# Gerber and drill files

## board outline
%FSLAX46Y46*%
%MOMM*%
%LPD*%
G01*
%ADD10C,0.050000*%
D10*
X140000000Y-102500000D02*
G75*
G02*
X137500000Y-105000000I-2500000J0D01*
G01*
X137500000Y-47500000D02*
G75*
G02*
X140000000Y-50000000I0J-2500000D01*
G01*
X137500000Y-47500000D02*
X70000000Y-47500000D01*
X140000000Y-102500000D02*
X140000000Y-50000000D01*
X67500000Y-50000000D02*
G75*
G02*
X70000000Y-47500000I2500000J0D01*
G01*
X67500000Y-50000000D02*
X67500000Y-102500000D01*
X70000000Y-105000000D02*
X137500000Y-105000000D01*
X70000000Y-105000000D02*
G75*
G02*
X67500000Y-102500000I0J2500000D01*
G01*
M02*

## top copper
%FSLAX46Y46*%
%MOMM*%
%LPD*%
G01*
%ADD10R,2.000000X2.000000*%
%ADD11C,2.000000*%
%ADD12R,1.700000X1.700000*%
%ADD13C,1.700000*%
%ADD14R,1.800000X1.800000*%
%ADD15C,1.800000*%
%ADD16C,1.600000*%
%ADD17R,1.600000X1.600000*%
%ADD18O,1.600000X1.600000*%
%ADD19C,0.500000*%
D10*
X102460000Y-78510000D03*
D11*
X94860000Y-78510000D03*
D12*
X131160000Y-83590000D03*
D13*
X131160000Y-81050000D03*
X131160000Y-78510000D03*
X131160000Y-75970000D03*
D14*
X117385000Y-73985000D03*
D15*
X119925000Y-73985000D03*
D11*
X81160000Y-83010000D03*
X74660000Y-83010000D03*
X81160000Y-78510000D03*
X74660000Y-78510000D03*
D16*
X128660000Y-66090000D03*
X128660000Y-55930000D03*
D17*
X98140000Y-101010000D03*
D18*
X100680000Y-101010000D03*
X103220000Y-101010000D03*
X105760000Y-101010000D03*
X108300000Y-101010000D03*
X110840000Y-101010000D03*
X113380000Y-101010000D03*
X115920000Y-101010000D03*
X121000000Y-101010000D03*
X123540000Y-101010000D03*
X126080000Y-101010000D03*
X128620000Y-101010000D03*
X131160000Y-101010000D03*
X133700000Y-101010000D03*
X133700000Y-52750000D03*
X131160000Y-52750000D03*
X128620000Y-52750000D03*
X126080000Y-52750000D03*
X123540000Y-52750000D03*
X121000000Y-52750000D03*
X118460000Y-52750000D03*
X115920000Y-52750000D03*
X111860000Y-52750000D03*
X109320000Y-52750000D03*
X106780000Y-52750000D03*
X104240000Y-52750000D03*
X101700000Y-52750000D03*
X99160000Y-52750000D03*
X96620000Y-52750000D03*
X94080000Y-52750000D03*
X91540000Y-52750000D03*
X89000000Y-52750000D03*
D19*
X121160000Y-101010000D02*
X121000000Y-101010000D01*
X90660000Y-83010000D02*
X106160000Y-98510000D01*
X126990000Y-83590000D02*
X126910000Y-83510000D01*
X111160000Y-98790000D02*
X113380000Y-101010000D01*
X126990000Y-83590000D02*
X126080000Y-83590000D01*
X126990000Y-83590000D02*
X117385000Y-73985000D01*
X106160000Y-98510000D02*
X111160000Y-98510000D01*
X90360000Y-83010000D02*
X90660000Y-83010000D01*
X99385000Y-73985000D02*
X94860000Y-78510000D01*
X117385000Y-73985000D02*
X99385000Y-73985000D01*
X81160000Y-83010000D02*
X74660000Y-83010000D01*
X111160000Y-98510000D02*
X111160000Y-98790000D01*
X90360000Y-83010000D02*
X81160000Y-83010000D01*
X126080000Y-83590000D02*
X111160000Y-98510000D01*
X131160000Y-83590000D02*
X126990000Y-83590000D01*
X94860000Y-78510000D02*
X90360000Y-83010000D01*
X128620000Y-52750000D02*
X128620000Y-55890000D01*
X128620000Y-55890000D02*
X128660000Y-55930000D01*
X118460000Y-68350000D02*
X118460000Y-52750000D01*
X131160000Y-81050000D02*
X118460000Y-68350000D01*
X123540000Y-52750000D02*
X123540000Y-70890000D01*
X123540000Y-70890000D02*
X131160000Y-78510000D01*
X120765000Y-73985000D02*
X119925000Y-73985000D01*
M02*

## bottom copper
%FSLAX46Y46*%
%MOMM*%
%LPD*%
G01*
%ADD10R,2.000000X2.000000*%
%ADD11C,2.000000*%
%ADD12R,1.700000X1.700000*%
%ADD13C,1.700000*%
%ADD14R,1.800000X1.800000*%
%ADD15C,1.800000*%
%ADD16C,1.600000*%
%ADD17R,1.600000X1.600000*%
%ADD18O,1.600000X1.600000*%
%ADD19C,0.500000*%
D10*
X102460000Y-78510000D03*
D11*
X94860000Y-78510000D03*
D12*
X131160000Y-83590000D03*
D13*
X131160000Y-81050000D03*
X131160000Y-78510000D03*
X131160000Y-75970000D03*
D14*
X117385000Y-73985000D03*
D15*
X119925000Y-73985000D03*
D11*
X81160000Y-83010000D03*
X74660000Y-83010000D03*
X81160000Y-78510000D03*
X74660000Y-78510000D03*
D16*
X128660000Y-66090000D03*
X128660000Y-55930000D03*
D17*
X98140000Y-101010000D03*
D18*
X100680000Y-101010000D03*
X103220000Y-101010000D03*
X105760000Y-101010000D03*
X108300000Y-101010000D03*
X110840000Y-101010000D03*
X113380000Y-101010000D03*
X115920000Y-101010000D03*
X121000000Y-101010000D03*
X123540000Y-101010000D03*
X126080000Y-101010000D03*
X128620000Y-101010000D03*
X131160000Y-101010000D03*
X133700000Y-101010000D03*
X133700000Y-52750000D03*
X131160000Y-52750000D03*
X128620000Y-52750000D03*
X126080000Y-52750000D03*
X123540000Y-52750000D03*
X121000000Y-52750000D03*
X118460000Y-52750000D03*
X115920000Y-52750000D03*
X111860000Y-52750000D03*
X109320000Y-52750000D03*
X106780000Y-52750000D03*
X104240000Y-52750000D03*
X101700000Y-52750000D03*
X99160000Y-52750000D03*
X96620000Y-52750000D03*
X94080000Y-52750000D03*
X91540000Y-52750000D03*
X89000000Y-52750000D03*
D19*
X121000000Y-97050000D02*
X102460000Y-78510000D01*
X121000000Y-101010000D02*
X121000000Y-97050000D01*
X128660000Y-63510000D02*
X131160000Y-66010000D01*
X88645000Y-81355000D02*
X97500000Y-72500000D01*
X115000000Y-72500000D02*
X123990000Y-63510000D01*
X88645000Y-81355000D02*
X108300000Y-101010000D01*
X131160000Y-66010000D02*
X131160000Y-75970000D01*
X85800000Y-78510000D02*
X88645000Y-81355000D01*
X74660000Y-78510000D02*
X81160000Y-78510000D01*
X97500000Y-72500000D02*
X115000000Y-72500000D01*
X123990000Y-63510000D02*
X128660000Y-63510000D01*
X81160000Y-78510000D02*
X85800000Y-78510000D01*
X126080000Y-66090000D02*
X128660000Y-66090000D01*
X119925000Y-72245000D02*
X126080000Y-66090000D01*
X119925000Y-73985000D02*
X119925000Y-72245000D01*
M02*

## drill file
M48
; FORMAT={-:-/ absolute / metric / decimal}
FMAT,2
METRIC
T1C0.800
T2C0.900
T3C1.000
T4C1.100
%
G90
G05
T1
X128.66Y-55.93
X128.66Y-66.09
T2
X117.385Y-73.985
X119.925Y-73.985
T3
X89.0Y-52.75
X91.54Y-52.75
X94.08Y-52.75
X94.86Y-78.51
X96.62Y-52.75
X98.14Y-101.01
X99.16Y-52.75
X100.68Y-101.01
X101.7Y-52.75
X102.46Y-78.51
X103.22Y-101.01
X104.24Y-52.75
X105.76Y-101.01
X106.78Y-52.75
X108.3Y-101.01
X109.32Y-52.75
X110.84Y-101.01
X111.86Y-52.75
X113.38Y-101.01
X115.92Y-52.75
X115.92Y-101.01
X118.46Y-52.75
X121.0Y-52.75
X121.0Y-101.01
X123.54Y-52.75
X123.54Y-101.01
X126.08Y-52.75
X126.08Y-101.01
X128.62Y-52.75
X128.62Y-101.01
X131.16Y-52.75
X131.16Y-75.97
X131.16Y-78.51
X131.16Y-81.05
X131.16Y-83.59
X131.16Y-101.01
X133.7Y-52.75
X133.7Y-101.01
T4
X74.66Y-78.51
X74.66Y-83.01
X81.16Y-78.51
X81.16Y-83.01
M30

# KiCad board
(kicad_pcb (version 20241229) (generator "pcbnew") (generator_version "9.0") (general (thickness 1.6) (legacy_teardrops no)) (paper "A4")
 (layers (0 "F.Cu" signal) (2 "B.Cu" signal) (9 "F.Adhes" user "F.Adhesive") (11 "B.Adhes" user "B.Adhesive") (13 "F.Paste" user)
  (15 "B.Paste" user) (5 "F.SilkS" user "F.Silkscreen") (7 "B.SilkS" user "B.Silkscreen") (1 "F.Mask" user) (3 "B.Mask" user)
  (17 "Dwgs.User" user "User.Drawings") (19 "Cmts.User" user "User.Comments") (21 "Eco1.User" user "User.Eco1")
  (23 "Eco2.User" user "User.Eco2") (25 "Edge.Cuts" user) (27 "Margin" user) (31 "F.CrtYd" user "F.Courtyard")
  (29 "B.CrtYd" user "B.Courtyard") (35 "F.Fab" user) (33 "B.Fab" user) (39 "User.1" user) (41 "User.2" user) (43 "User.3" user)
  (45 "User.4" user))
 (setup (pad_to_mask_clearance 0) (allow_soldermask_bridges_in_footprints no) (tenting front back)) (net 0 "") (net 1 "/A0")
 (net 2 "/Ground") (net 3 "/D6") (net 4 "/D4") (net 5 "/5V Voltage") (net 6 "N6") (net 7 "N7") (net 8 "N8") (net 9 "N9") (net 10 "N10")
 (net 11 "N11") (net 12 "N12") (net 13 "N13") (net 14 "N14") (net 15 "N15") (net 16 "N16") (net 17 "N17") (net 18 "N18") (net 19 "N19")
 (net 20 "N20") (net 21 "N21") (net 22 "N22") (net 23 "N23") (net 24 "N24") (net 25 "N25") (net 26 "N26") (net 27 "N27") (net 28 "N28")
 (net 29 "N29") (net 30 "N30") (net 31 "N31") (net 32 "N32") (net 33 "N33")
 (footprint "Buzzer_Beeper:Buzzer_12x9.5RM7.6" (layer "F.Cu") (at 102.46 78.51 180)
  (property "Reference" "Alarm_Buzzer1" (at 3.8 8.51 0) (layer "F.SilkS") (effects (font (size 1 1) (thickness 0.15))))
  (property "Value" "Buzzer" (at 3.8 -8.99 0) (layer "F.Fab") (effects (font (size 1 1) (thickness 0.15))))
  (pad "1" thru_hole rect (at 0 0 180) (size 2 2) (drill 1) (layers "*.Cu" "*.Mask") (remove_unused_layers no) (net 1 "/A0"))
  (pad "2" thru_hole circle (at 7.6 0 180) (size 2 2) (drill 1) (layers "*.Cu" "*.Mask") (remove_unused_layers no) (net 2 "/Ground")))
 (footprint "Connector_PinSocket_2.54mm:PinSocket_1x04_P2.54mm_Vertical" (layer "F.Cu") (at 131.16 83.59 180)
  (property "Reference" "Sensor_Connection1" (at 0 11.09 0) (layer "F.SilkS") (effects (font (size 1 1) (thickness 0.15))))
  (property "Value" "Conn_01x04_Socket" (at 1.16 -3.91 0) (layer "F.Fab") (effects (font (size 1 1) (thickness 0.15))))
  (pad "1" thru_hole rect (at 0 0 180) (size 1.7 1.7) (drill 1) (layers "*.Cu" "*.Mask") (remove_unused_layers no) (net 2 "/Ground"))
  (pad "2" thru_hole circle (at 0 2.54 180) (size 1.7 1.7) (drill 1) (layers "*.Cu" "*.Mask") (remove_unused_layers no) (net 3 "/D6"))
  (pad "3" thru_hole circle (at 0 5.08 180) (size 1.7 1.7) (drill 1) (layers "*.Cu" "*.Mask") (remove_unused_layers no) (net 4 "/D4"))
  (pad "4" thru_hole circle (at 0 7.62 180) (size 1.7 1.7) (drill 1) (layers "*.Cu" "*.Mask") (remove_unused_layers no)
   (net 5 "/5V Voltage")))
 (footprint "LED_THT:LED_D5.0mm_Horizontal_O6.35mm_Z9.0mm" (layer "F.Cu") (at 117.385 73.985)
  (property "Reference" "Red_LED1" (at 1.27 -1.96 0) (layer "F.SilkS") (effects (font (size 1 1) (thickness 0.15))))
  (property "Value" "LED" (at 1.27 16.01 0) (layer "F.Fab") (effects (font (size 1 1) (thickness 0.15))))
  (pad "1" thru_hole rect (at 0 0) (size 1.8 1.8) (drill 0.9) (layers "*.Cu" "*.Mask") (remove_unused_layers no) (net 2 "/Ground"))
  (pad "2" thru_hole circle (at 2.54 0) (size 1.8 1.8) (drill 0.9) (layers "*.Cu" "*.Mask") (remove_unused_layers no) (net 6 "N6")))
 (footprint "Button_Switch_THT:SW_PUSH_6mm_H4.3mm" (layer "F.Cu") (at 81.16 83.01 180)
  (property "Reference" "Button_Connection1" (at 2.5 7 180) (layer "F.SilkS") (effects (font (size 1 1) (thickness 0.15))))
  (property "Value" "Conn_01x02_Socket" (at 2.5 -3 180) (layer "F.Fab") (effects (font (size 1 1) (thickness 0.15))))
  (pad "1" thru_hole circle (at 0 0 270) (size 2 2) (drill 1.1) (layers "*.Cu" "*.Mask") (remove_unused_layers no) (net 2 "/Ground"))
  (pad "1" thru_hole circle (at 6.5 0 270) (size 2 2) (drill 1.1) (layers "*.Cu" "*.Mask") (remove_unused_layers no) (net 2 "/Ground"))
  (pad "2" thru_hole circle (at 0 4.5 270) (size 2 2) (drill 1.1) (layers "*.Cu" "*.Mask") (remove_unused_layers no) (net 5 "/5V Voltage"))
  (pad "2" thru_hole circle (at 6.5 4.5 270) (size 2 2) (drill 1.1) (layers "*.Cu" "*.Mask") (remove_unused_layers no) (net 5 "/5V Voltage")))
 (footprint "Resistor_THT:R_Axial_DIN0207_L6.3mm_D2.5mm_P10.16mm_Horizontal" (layer "F.Cu") (at 128.66 66.09 90)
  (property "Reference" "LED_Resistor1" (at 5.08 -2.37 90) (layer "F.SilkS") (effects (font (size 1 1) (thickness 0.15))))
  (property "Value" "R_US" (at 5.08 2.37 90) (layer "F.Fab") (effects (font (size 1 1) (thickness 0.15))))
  (pad "1" thru_hole circle (at 0 0 90) (size 1.6 1.6) (drill 0.8) (layers "*.Cu" "*.Mask") (remove_unused_layers no) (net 6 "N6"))
  (pad "2" thru_hole circle (at 10.16 0 90) (size 1.6 1.6) (drill 0.8) (layers "*.Cu" "*.Mask") (remove_unused_layers no) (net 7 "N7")))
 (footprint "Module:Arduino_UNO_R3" (layer "B.Cu") (at 98.14 101.01)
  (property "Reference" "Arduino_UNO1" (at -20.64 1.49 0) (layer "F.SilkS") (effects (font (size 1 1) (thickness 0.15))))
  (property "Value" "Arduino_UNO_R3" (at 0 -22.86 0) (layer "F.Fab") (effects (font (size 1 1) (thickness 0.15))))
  (pad "1" thru_hole rect (at 0 0 270) (size 1.6 1.6) (drill 1) (layers "*.Cu" "*.Mask") (remove_unused_layers no) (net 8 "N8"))
  (pad "2" thru_hole oval (at 2.54 0 270) (size 1.6 1.6) (drill 1) (layers "*.Cu" "*.Mask") (remove_unused_layers no) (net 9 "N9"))
  (pad "3" thru_hole oval (at 5.08 0 270) (size 1.6 1.6) (drill 1) (layers "*.Cu" "*.Mask") (remove_unused_layers no) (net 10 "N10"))
  (pad "4" thru_hole oval (at 7.62 0 270) (size 1.6 1.6) (drill 1) (layers "*.Cu" "*.Mask") (remove_unused_layers no) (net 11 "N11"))
  (pad "5" thru_hole oval (at 10.16 0 270) (size 1.6 1.6) (drill 1) (layers "*.Cu" "*.Mask") (remove_unused_layers no) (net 5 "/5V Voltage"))
  (pad "6" thru_hole oval (at 12.7 0 270) (size 1.6 1.6) (drill 1) (layers "*.Cu" "*.Mask") (remove_unused_layers no) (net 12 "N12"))
  (pad "7" thru_hole oval (at 15.24 0 270) (size 1.6 1.6) (drill 1) (layers "*.Cu" "*.Mask") (remove_unused_layers no) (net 2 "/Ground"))
  (pad "8" thru_hole oval (at 17.78 0 270) (size 1.6 1.6) (drill 1) (layers "*.Cu" "*.Mask") (remove_unused_layers no) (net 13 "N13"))
  (pad "9" thru_hole oval (at 22.86 0 270) (size 1.6 1.6) (drill 1) (layers "*.Cu" "*.Mask") (remove_unused_layers no) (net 1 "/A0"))
  (pad "10" thru_hole oval (at 25.4 0 270) (size 1.6 1.6) (drill 1) (layers "*.Cu" "*.Mask") (remove_unused_layers no) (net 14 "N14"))
  (pad "11" thru_hole oval (at 27.94 0 270) (size 1.6 1.6) (drill 1) (layers "*.Cu" "*.Mask") (remove_unused_layers no) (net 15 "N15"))
  (pad "12" thru_hole oval (at 30.48 0 270) (size 1.6 1.6) (drill 1) (layers "*.Cu" "*.Mask") (remove_unused_layers no) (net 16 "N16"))
  (pad "13" thru_hole oval (at 33.02 0 270) (size 1.6 1.6) (drill 1) (layers "*.Cu" "*.Mask") (remove_unused_layers no) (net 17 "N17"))
  (pad "14" thru_hole oval (at 35.56 0 270) (size 1.6 1.6) (drill 1) (layers "*.Cu" "*.Mask") (remove_unused_layers no) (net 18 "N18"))
  (pad "15" thru_hole oval (at 35.56 -48.26 270) (size 1.6 1.6) (drill 1) (layers "*.Cu" "*.Mask") (remove_unused_layers no) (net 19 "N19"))
  (pad "16" thru_hole oval (at 33.02 -48.26 270) (size 1.6 1.6) (drill 1) (layers "*.Cu" "*.Mask") (remove_unused_layers no) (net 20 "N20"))
  (pad "17" thru_hole oval (at 30.48 -48.26 270) (size 1.6 1.6) (drill 1) (layers "*.Cu" "*.Mask") (remove_unused_layers no) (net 7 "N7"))
  (pad "18" thru_hole oval (at 27.94 -48.26 270) (size 1.6 1.6) (drill 1) (layers "*.Cu" "*.Mask") (remove_unused_layers no) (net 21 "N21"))
  (pad "19" thru_hole oval (at 25.4 -48.26 270) (size 1.6 1.6) (drill 1) (layers "*.Cu" "*.Mask") (remove_unused_layers no) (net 4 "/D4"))
  (pad "20" thru_hole oval (at 22.86 -48.26 270) (size 1.6 1.6) (drill 1) (layers "*.Cu" "*.Mask") (remove_unused_layers no) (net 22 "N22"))
  (pad "21" thru_hole oval (at 20.32 -48.26 270) (size 1.6 1.6) (drill 1) (layers "*.Cu" "*.Mask") (remove_unused_layers no) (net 3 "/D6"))
  (pad "22" thru_hole oval (at 17.78 -48.26 270) (size 1.6 1.6) (drill 1) (layers "*.Cu" "*.Mask") (remove_unused_layers no) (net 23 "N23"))
  (pad "23" thru_hole oval (at 13.72 -48.26 270) (size 1.6 1.6) (drill 1) (layers "*.Cu" "*.Mask") (remove_unused_layers no) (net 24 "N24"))
  (pad "24" thru_hole oval (at 11.18 -48.26 270) (size 1.6 1.6) (drill 1) (layers "*.Cu" "*.Mask") (remove_unused_layers no) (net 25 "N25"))
  (pad "25" thru_hole oval (at 8.64 -48.26 270) (size 1.6 1.6) (drill 1) (layers "*.Cu" "*.Mask") (remove_unused_layers no) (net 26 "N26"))
  (pad "26" thru_hole oval (at 6.1 -48.26 270) (size 1.6 1.6) (drill 1) (layers "*.Cu" "*.Mask") (remove_unused_layers no) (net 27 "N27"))
  (pad "27" thru_hole oval (at 3.56 -48.26 270) (size 1.6 1.6) (drill 1) (layers "*.Cu" "*.Mask") (remove_unused_layers no) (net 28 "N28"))
  (pad "28" thru_hole oval (at 1.02 -48.26 270) (size 1.6 1.6) (drill 1) (layers "*.Cu" "*.Mask") (remove_unused_layers no) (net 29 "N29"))
  (pad "29" thru_hole oval (at -1.52 -48.26 270) (size 1.6 1.6) (drill 1) (layers "*.Cu" "*.Mask") (remove_unused_layers no) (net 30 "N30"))
  (pad "30" thru_hole oval (at -4.06 -48.26 270) (size 1.6 1.6) (drill 1) (layers "*.Cu" "*.Mask") (remove_unused_layers no) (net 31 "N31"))
  (pad "31" thru_hole oval (at -6.6 -48.26 270) (size 1.6 1.6) (drill 1) (layers "*.Cu" "*.Mask") (remove_unused_layers no) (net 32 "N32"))
  (pad "32" thru_hole oval (at -9.14 -48.26 270) (size 1.6 1.6) (drill 1) (layers "*.Cu" "*.Mask") (remove_unused_layers no) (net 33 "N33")))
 (gr_arc (start 140 102.5) (mid 139.267767 104.267767) (end 137.5 105) (stroke (width 0.05) (type default)) (layer "Edge.Cuts"))
 (gr_arc (start 137.5 47.5) (mid 139.267767 48.232233) (end 140 50) (stroke (width 0.05) (type default)) (layer "Edge.Cuts"))
 (gr_line (start 137.5 47.5) (end 70 47.5) (stroke (width 0.05) (type default)) (layer "Edge.Cuts"))
 (gr_line (start 140 102.5) (end 140 50) (stroke (width 0.05) (type default)) (layer "Edge.Cuts"))
 (gr_arc (start 67.5 50) (mid 68.232233 48.232233) (end 70 47.5) (stroke (width 0.05) (type default)) (layer "Edge.Cuts"))
 (gr_line (start 67.5 50) (end 67.5 102.5) (stroke (width 0.05) (type default)) (layer "Edge.Cuts"))
 (gr_line (start 70 105) (end 137.5 105) (stroke (width 0.05) (type default)) (layer "Edge.Cuts"))
 (gr_arc (start 70 105) (mid 68.232233 104.267767) (end 67.5 102.5) (stroke (width 0.05) (type default)) (layer "Edge.Cuts"))
 (segment (start 121.16 101.01) (end 121 101.01) (width 0.5) (layer "F.Cu") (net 1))
 (segment (start 121 97.05) (end 102.46 78.51) (width 0.5) (layer "B.Cu") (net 1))
 (segment (start 121 101.01) (end 121 97.05) (width 0.5) (layer "B.Cu") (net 1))
 (segment (start 90.66 83.01) (end 106.16 98.51) (width 0.5) (layer "F.Cu") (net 2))
 (segment (start 126.99 83.59) (end 126.91 83.51) (width 0.5) (layer "F.Cu") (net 2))
 (segment (start 111.16 98.79) (end 113.38 101.01) (width 0.5) (layer "F.Cu") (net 2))
 (segment (start 126.99 83.59) (end 126.08 83.59) (width 0.5) (layer "F.Cu") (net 2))
 (segment (start 126.99 83.59) (end 117.385 73.985) (width 0.5) (layer "F.Cu") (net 2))
 (segment (start 106.16 98.51) (end 111.16 98.51) (width 0.5) (layer "F.Cu") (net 2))
 (segment (start 90.36 83.01) (end 90.66 83.01) (width 0.5) (layer "F.Cu") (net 2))
 (segment (start 99.385 73.985) (end 94.86 78.51) (width 0.5) (layer "F.Cu") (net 2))
 (segment (start 117.385 73.985) (end 99.385 73.985) (width 0.5) (layer "F.Cu") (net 2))
 (segment (start 81.16 83.01) (end 74.66 83.01) (width 0.5) (layer "F.Cu") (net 2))
 (segment (start 111.16 98.51) (end 111.16 98.79) (width 0.5) (layer "F.Cu") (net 2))
 (segment (start 90.36 83.01) (end 81.16 83.01) (width 0.5) (layer "F.Cu") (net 2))
 (segment (start 126.08 83.59) (end 111.16 98.51) (width 0.5) (layer "F.Cu") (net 2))
 (segment (start 131.16 83.59) (end 126.99 83.59) (width 0.5) (layer "F.Cu") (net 2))
 (segment (start 94.86 78.51) (end 90.36 83.01) (width 0.5) (layer "F.Cu") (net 2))
 (segment (start 128.62 52.75) (end 128.62 55.89) (width 0.5) (layer "F.Cu") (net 7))
 (segment (start 128.62 55.89) (end 128.66 55.93) (width 0.5) (layer "F.Cu") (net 7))
 (segment (start 128.66 63.51) (end 131.16 66.01) (width 0.5) (layer "B.Cu") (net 5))
 (segment (start 88.645 81.355) (end 97.5 72.5) (width 0.5) (layer "B.Cu") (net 5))
 (segment (start 115 72.5) (end 123.99 63.51) (width 0.5) (layer "B.Cu") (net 5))
 (segment (start 88.645 81.355) (end 108.3 101.01) (width 0.5) (layer "B.Cu") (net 5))
 (segment (start 131.16 66.01) (end 131.16 75.97) (width 0.5) (layer "B.Cu") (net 5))
 (segment (start 85.8 78.51) (end 88.645 81.355) (width 0.5) (layer "B.Cu") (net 5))
 (segment (start 74.66 78.51) (end 81.16 78.51) (width 0.5) (layer "B.Cu") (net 5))
 (segment (start 97.5 72.5) (end 115 72.5) (width 0.5) (layer "B.Cu") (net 5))
 (segment (start 123.99 63.51) (end 128.66 63.51) (width 0.5) (layer "B.Cu") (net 5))
 (segment (start 81.16 78.51) (end 85.8 78.51) (width 0.5) (layer "B.Cu") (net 5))
 (segment (start 118.46 68.35) (end 118.46 52.75) (width 0.5) (layer "F.Cu") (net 3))
 (segment (start 131.16 81.05) (end 118.46 68.35) (width 0.5) (layer "F.Cu") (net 3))
 (segment (start 123.54 52.75) (end 123.54 70.89) (width 0.5) (layer "F.Cu") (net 4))
 (segment (start 123.54 70.89) (end 131.16 78.51) (width 0.5) (layer "F.Cu") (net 4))
 (segment (start 120.765 73.985) (end 119.925 73.985) (width 0.5) (layer "F.Cu") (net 6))
 (segment (start 126.08 66.09) (end 128.66 66.09) (width 0.5) (layer "B.Cu") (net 6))
 (segment (start 119.925 72.245) (end 126.08 66.09) (width 0.5) (layer "B.Cu") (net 6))
 (segment (start 119.925 73.985) (end 119.925 72.245) (width 0.5) (layer "B.Cu") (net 6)))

